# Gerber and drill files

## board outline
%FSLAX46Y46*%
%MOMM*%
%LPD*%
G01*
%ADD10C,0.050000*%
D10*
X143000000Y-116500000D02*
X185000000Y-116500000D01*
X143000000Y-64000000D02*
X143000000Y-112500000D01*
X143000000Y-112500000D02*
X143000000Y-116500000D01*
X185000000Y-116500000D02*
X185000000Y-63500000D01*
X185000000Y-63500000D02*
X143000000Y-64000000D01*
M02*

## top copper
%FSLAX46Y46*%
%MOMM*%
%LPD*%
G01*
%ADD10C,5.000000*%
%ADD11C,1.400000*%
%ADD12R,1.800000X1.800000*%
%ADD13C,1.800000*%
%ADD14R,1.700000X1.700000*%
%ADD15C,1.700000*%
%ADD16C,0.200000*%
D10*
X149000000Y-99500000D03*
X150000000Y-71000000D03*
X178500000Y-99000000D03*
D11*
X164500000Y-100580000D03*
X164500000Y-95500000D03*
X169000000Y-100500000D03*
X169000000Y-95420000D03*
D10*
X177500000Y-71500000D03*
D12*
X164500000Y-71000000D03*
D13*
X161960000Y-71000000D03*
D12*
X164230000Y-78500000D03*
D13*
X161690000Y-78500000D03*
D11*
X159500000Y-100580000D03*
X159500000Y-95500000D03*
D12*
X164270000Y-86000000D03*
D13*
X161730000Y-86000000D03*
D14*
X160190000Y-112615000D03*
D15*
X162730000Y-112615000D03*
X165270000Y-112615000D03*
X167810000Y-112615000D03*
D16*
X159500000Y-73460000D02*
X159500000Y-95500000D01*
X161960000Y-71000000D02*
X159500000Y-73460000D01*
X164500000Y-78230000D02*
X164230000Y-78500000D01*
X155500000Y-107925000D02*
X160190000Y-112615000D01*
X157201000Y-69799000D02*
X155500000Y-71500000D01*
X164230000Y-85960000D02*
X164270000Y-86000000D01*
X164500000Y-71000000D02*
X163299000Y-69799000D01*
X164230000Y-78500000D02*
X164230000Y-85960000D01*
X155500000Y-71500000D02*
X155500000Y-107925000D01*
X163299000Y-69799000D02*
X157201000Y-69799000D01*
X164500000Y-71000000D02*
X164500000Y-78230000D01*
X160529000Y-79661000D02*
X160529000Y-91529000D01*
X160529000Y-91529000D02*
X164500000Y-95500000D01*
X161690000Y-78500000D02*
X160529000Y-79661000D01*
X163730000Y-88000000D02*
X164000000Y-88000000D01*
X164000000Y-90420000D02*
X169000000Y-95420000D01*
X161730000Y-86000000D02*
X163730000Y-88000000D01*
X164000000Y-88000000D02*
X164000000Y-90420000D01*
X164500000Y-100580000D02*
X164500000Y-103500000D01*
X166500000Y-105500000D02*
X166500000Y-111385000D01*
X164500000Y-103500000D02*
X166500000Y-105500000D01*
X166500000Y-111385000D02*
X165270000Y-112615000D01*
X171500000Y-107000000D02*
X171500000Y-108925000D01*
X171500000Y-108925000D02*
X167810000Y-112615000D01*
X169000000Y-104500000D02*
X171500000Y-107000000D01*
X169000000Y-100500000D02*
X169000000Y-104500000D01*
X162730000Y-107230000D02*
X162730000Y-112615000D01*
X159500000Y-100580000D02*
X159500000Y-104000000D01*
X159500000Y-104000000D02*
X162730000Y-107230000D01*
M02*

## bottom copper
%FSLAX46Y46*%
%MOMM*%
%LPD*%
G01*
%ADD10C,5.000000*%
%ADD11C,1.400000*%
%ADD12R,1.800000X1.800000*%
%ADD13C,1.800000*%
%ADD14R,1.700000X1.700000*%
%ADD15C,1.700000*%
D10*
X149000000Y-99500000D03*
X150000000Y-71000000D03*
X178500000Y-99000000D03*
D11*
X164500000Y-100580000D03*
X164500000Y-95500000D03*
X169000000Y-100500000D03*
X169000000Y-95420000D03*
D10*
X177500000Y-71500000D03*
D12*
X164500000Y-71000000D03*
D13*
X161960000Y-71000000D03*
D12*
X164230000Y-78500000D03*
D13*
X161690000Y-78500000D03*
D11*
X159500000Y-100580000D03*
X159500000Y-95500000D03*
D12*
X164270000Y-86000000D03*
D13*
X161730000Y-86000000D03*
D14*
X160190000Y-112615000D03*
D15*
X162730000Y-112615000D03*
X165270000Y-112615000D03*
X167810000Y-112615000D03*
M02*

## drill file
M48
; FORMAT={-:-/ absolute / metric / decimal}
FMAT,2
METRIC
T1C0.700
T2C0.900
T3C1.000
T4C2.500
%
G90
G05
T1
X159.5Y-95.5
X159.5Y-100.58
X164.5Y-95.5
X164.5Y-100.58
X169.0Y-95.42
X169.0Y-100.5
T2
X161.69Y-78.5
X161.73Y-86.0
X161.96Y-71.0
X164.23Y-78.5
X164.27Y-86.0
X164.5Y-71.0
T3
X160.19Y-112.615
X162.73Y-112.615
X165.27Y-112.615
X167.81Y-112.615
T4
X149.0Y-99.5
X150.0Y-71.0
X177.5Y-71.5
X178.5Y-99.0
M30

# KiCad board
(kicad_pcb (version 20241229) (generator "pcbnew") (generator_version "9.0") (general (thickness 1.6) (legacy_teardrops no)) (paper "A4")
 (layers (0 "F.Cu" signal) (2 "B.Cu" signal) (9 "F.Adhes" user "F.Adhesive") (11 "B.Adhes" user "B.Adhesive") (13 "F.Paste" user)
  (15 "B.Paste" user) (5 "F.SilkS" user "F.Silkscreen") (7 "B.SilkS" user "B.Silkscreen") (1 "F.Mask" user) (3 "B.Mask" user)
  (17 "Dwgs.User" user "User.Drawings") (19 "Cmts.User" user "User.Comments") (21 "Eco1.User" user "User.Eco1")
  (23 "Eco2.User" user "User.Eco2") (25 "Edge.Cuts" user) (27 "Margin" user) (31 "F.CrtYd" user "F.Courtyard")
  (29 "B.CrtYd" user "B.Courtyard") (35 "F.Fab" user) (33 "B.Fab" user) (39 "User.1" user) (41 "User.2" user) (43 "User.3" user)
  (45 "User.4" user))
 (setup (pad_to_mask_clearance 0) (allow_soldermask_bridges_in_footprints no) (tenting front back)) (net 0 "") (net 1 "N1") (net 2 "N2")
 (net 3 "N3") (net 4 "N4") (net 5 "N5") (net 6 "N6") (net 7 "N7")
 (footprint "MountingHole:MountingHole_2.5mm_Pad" (layer "F.Cu") (at 149 99.5)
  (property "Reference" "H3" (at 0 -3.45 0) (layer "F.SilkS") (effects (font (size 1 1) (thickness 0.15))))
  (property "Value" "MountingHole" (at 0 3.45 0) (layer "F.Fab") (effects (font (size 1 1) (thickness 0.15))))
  (pad "1" thru_hole circle (at 0 0) (size 5 5) (drill 2.5) (layers "*.Cu" "*.Mask") (remove_unused_layers no) (zone_connect 2)))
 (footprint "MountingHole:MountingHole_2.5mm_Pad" (layer "F.Cu") (at 150 71)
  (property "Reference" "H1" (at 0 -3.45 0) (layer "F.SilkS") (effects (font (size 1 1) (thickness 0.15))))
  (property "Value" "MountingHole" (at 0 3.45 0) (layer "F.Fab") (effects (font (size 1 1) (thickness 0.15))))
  (pad "1" thru_hole circle (at 0 0) (size 5 5) (drill 2.5) (layers "*.Cu" "*.Mask") (remove_unused_layers no) (zone_connect 2)))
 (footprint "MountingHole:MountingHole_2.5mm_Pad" (layer "F.Cu") (at 178.5 99)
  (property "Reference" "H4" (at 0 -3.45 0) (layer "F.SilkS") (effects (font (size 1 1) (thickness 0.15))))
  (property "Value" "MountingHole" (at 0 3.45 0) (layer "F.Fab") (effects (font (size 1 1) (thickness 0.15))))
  (pad "1" thru_hole circle (at 0 0) (size 5 5) (drill 2.5) (layers "*.Cu" "*.Mask") (remove_unused_layers no) (zone_connect 2)))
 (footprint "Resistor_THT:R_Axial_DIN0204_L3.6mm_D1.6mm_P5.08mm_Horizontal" (layer "F.Cu") (at 164.5 100.58 90)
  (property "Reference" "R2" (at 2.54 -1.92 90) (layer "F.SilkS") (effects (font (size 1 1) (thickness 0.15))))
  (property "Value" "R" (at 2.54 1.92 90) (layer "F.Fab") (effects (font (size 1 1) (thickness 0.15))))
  (pad "1" thru_hole circle (at 0 0 90) (size 1.4 1.4) (drill 0.7) (layers "*.Cu" "*.Mask") (remove_unused_layers no) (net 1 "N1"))
  (pad "2" thru_hole circle (at 5.08 0 90) (size 1.4 1.4) (drill 0.7) (layers "*.Cu" "*.Mask") (remove_unused_layers no) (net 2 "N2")))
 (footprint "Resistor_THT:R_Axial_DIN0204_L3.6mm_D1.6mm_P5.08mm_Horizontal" (layer "F.Cu") (at 169 100.5 90)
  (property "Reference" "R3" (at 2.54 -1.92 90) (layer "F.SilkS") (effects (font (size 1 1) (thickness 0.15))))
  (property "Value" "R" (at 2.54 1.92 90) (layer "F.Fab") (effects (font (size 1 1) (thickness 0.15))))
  (pad "1" thru_hole circle (at 0 0 90) (size 1.4 1.4) (drill 0.7) (layers "*.Cu" "*.Mask") (remove_unused_layers no) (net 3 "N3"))
  (pad "2" thru_hole circle (at 5.08 0 90) (size 1.4 1.4) (drill 0.7) (layers "*.Cu" "*.Mask") (remove_unused_layers no) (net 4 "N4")))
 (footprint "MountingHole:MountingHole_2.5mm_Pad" (layer "F.Cu") (at 177.5 71.5)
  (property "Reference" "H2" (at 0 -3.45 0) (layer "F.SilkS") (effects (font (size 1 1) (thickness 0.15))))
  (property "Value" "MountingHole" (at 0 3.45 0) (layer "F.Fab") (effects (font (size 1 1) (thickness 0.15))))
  (pad "1" thru_hole circle (at 0 0) (size 5 5) (drill 2.5) (layers "*.Cu" "*.Mask") (remove_unused_layers no) (zone_connect 2)))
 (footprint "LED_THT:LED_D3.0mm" (layer "F.Cu") (at 164.5 71 180)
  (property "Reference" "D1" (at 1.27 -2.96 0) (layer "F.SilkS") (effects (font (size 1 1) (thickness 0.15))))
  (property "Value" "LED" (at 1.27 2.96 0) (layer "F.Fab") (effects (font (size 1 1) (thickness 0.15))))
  (pad "1" thru_hole rect (at 0 0 180) (size 1.8 1.8) (drill 0.9) (layers "*.Cu" "*.Mask") (remove_unused_layers no) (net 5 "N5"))
  (pad "2" thru_hole circle (at 2.54 0 180) (size 1.8 1.8) (drill 0.9) (layers "*.Cu" "*.Mask") (remove_unused_layers no) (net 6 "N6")))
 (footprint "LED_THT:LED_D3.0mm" (layer "F.Cu") (at 164.23 78.5 180)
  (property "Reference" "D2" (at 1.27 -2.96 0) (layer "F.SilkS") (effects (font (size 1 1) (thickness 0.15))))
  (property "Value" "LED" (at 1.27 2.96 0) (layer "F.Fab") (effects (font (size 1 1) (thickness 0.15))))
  (pad "1" thru_hole rect (at 0 0 180) (size 1.8 1.8) (drill 0.9) (layers "*.Cu" "*.Mask") (remove_unused_layers no) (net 5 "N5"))
  (pad "2" thru_hole circle (at 2.54 0 180) (size 1.8 1.8) (drill 0.9) (layers "*.Cu" "*.Mask") (remove_unused_layers no) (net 2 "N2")))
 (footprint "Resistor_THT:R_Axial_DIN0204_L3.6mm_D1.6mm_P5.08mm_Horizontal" (layer "F.Cu") (at 159.5 100.58 90)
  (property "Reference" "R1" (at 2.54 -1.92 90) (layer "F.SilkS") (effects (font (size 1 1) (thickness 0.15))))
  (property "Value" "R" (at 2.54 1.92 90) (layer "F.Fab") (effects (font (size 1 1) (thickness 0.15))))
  (pad "1" thru_hole circle (at 0 0 90) (size 1.4 1.4) (drill 0.7) (layers "*.Cu" "*.Mask") (remove_unused_layers no) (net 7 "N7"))
  (pad "2" thru_hole circle (at 5.08 0 90) (size 1.4 1.4) (drill 0.7) (layers "*.Cu" "*.Mask") (remove_unused_layers no) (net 6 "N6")))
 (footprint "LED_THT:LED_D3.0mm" (layer "F.Cu") (at 164.27 86 180)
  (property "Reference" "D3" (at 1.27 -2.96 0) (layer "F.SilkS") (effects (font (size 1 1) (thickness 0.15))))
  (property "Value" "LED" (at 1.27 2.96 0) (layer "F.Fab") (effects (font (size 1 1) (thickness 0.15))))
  (pad "1" thru_hole rect (at 0 0 180) (size 1.8 1.8) (drill 0.9) (layers "*.Cu" "*.Mask") (remove_unused_layers no) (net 5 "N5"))
  (pad "2" thru_hole circle (at 2.54 0 180) (size 1.8 1.8) (drill 0.9) (layers "*.Cu" "*.Mask") (remove_unused_layers no) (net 4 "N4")))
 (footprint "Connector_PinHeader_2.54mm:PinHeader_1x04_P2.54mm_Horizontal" (layer "B.Cu") (at 160.19 112.615 -90)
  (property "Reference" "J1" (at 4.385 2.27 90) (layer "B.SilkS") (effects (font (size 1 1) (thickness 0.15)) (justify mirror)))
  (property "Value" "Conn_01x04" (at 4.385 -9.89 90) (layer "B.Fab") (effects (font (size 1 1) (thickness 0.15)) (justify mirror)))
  (pad "1" thru_hole rect (at 0 0 270) (size 1.7 1.7) (drill 1) (layers "*.Cu" "*.Mask") (remove_unused_layers no) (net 5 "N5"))
  (pad "2" thru_hole circle (at 0 -2.54 270) (size 1.7 1.7) (drill 1) (layers "*.Cu" "*.Mask") (remove_unused_layers no) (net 7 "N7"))
  (pad "3" thru_hole circle (at 0 -5.08 270) (size 1.7 1.7) (drill 1) (layers "*.Cu" "*.Mask") (remove_unused_layers no) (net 1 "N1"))
  (pad "4" thru_hole circle (at 0 -7.62 270) (size 1.7 1.7) (drill 1) (layers "*.Cu" "*.Mask") (remove_unused_layers no) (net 3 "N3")))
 (gr_line (start 143 116.5) (end 185 116.5) (stroke (width 0.05) (type default)) (layer "Edge.Cuts"))
 (gr_line (start 143 64) (end 143 112.5) (stroke (width 0.05) (type default)) (layer "Edge.Cuts"))
 (gr_line (start 143 112.5) (end 143 116.5) (stroke (width 0.05) (type default)) (layer "Edge.Cuts"))
 (gr_line (start 185 116.5) (end 185 63.5) (stroke (width 0.05) (type default)) (layer "Edge.Cuts"))
 (gr_line (start 185 63.5) (end 143 64) (stroke (width 0.05) (type default)) (layer "Edge.Cuts"))
 (segment (start 159.5 73.46) (end 159.5 95.5) (width 0.2) (layer "F.Cu") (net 6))
 (segment (start 161.96 71) (end 159.5 73.46) (width 0.2) (layer "F.Cu") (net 6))
 (segment (start 164.5 78.23) (end 164.23 78.5) (width 0.2) (layer "F.Cu") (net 5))
 (segment (start 155.5 107.925) (end 160.19 112.615) (width 0.2) (layer "F.Cu") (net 5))
 (segment (start 157.201 69.799) (end 155.5 71.5) (width 0.2) (layer "F.Cu") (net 5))
 (segment (start 164.23 85.96) (end 164.27 86) (width 0.2) (layer "F.Cu") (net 5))
 (segment (start 164.5 71) (end 163.299 69.799) (width 0.2) (layer "F.Cu") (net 5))
 (segment (start 164.23 78.5) (end 164.23 85.96) (width 0.2) (layer "F.Cu") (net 5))
 (segment (start 155.5 71.5) (end 155.5 107.925) (width 0.2) (layer "F.Cu") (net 5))
 (segment (start 163.299 69.799) (end 157.201 69.799) (width 0.2) (layer "F.Cu") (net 5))
 (segment (start 164.5 71) (end 164.5 78.23) (width 0.2) (layer "F.Cu") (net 5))
 (segment (start 160.529 79.661) (end 160.529 91.529) (width 0.2) (layer "F.Cu") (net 2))
 (segment (start 160.529 91.529) (end 164.5 95.5) (width 0.2) (layer "F.Cu") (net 2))
 (segment (start 161.69 78.5) (end 160.529 79.661) (width 0.2) (layer "F.Cu") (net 2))
 (segment (start 163.73 88) (end 164 88) (width 0.2) (layer "F.Cu") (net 4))
 (segment (start 164 90.42) (end 169 95.42) (width 0.2) (layer "F.Cu") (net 4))
 (segment (start 161.73 86) (end 163.73 88) (width 0.2) (layer "F.Cu") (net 4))
 (segment (start 164 88) (end 164 90.42) (width 0.2) (layer "F.Cu") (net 4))
 (segment (start 164.5 100.58) (end 164.5 103.5) (width 0.2) (layer "F.Cu") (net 1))
 (segment (start 166.5 105.5) (end 166.5 111.385) (width 0.2) (layer "F.Cu") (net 1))
 (segment (start 164.5 103.5) (end 166.5 105.5) (width 0.2) (layer "F.Cu") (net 1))
 (segment (start 166.5 111.385) (end 165.27 112.615) (width 0.2) (layer "F.Cu") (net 1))
 (segment (start 171.5 107) (end 171.5 108.925) (width 0.2) (layer "F.Cu") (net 3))
 (segment (start 171.5 108.925) (end 167.81 112.615) (width 0.2) (layer "F.Cu") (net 3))
 (segment (start 169 104.5) (end 171.5 107) (width 0.2) (layer "F.Cu") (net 3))
 (segment (start 169 100.5) (end 169 104.5) (width 0.2) (layer "F.Cu") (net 3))
 (segment (start 162.73 107.23) (end 162.73 112.615) (width 0.2) (layer "F.Cu") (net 7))
 (segment (start 159.5 100.58) (end 159.5 104) (width 0.2) (layer "F.Cu") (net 7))
 (segment (start 159.5 104) (end 162.73 107.23) (width 0.2) (layer "F.Cu") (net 7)))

